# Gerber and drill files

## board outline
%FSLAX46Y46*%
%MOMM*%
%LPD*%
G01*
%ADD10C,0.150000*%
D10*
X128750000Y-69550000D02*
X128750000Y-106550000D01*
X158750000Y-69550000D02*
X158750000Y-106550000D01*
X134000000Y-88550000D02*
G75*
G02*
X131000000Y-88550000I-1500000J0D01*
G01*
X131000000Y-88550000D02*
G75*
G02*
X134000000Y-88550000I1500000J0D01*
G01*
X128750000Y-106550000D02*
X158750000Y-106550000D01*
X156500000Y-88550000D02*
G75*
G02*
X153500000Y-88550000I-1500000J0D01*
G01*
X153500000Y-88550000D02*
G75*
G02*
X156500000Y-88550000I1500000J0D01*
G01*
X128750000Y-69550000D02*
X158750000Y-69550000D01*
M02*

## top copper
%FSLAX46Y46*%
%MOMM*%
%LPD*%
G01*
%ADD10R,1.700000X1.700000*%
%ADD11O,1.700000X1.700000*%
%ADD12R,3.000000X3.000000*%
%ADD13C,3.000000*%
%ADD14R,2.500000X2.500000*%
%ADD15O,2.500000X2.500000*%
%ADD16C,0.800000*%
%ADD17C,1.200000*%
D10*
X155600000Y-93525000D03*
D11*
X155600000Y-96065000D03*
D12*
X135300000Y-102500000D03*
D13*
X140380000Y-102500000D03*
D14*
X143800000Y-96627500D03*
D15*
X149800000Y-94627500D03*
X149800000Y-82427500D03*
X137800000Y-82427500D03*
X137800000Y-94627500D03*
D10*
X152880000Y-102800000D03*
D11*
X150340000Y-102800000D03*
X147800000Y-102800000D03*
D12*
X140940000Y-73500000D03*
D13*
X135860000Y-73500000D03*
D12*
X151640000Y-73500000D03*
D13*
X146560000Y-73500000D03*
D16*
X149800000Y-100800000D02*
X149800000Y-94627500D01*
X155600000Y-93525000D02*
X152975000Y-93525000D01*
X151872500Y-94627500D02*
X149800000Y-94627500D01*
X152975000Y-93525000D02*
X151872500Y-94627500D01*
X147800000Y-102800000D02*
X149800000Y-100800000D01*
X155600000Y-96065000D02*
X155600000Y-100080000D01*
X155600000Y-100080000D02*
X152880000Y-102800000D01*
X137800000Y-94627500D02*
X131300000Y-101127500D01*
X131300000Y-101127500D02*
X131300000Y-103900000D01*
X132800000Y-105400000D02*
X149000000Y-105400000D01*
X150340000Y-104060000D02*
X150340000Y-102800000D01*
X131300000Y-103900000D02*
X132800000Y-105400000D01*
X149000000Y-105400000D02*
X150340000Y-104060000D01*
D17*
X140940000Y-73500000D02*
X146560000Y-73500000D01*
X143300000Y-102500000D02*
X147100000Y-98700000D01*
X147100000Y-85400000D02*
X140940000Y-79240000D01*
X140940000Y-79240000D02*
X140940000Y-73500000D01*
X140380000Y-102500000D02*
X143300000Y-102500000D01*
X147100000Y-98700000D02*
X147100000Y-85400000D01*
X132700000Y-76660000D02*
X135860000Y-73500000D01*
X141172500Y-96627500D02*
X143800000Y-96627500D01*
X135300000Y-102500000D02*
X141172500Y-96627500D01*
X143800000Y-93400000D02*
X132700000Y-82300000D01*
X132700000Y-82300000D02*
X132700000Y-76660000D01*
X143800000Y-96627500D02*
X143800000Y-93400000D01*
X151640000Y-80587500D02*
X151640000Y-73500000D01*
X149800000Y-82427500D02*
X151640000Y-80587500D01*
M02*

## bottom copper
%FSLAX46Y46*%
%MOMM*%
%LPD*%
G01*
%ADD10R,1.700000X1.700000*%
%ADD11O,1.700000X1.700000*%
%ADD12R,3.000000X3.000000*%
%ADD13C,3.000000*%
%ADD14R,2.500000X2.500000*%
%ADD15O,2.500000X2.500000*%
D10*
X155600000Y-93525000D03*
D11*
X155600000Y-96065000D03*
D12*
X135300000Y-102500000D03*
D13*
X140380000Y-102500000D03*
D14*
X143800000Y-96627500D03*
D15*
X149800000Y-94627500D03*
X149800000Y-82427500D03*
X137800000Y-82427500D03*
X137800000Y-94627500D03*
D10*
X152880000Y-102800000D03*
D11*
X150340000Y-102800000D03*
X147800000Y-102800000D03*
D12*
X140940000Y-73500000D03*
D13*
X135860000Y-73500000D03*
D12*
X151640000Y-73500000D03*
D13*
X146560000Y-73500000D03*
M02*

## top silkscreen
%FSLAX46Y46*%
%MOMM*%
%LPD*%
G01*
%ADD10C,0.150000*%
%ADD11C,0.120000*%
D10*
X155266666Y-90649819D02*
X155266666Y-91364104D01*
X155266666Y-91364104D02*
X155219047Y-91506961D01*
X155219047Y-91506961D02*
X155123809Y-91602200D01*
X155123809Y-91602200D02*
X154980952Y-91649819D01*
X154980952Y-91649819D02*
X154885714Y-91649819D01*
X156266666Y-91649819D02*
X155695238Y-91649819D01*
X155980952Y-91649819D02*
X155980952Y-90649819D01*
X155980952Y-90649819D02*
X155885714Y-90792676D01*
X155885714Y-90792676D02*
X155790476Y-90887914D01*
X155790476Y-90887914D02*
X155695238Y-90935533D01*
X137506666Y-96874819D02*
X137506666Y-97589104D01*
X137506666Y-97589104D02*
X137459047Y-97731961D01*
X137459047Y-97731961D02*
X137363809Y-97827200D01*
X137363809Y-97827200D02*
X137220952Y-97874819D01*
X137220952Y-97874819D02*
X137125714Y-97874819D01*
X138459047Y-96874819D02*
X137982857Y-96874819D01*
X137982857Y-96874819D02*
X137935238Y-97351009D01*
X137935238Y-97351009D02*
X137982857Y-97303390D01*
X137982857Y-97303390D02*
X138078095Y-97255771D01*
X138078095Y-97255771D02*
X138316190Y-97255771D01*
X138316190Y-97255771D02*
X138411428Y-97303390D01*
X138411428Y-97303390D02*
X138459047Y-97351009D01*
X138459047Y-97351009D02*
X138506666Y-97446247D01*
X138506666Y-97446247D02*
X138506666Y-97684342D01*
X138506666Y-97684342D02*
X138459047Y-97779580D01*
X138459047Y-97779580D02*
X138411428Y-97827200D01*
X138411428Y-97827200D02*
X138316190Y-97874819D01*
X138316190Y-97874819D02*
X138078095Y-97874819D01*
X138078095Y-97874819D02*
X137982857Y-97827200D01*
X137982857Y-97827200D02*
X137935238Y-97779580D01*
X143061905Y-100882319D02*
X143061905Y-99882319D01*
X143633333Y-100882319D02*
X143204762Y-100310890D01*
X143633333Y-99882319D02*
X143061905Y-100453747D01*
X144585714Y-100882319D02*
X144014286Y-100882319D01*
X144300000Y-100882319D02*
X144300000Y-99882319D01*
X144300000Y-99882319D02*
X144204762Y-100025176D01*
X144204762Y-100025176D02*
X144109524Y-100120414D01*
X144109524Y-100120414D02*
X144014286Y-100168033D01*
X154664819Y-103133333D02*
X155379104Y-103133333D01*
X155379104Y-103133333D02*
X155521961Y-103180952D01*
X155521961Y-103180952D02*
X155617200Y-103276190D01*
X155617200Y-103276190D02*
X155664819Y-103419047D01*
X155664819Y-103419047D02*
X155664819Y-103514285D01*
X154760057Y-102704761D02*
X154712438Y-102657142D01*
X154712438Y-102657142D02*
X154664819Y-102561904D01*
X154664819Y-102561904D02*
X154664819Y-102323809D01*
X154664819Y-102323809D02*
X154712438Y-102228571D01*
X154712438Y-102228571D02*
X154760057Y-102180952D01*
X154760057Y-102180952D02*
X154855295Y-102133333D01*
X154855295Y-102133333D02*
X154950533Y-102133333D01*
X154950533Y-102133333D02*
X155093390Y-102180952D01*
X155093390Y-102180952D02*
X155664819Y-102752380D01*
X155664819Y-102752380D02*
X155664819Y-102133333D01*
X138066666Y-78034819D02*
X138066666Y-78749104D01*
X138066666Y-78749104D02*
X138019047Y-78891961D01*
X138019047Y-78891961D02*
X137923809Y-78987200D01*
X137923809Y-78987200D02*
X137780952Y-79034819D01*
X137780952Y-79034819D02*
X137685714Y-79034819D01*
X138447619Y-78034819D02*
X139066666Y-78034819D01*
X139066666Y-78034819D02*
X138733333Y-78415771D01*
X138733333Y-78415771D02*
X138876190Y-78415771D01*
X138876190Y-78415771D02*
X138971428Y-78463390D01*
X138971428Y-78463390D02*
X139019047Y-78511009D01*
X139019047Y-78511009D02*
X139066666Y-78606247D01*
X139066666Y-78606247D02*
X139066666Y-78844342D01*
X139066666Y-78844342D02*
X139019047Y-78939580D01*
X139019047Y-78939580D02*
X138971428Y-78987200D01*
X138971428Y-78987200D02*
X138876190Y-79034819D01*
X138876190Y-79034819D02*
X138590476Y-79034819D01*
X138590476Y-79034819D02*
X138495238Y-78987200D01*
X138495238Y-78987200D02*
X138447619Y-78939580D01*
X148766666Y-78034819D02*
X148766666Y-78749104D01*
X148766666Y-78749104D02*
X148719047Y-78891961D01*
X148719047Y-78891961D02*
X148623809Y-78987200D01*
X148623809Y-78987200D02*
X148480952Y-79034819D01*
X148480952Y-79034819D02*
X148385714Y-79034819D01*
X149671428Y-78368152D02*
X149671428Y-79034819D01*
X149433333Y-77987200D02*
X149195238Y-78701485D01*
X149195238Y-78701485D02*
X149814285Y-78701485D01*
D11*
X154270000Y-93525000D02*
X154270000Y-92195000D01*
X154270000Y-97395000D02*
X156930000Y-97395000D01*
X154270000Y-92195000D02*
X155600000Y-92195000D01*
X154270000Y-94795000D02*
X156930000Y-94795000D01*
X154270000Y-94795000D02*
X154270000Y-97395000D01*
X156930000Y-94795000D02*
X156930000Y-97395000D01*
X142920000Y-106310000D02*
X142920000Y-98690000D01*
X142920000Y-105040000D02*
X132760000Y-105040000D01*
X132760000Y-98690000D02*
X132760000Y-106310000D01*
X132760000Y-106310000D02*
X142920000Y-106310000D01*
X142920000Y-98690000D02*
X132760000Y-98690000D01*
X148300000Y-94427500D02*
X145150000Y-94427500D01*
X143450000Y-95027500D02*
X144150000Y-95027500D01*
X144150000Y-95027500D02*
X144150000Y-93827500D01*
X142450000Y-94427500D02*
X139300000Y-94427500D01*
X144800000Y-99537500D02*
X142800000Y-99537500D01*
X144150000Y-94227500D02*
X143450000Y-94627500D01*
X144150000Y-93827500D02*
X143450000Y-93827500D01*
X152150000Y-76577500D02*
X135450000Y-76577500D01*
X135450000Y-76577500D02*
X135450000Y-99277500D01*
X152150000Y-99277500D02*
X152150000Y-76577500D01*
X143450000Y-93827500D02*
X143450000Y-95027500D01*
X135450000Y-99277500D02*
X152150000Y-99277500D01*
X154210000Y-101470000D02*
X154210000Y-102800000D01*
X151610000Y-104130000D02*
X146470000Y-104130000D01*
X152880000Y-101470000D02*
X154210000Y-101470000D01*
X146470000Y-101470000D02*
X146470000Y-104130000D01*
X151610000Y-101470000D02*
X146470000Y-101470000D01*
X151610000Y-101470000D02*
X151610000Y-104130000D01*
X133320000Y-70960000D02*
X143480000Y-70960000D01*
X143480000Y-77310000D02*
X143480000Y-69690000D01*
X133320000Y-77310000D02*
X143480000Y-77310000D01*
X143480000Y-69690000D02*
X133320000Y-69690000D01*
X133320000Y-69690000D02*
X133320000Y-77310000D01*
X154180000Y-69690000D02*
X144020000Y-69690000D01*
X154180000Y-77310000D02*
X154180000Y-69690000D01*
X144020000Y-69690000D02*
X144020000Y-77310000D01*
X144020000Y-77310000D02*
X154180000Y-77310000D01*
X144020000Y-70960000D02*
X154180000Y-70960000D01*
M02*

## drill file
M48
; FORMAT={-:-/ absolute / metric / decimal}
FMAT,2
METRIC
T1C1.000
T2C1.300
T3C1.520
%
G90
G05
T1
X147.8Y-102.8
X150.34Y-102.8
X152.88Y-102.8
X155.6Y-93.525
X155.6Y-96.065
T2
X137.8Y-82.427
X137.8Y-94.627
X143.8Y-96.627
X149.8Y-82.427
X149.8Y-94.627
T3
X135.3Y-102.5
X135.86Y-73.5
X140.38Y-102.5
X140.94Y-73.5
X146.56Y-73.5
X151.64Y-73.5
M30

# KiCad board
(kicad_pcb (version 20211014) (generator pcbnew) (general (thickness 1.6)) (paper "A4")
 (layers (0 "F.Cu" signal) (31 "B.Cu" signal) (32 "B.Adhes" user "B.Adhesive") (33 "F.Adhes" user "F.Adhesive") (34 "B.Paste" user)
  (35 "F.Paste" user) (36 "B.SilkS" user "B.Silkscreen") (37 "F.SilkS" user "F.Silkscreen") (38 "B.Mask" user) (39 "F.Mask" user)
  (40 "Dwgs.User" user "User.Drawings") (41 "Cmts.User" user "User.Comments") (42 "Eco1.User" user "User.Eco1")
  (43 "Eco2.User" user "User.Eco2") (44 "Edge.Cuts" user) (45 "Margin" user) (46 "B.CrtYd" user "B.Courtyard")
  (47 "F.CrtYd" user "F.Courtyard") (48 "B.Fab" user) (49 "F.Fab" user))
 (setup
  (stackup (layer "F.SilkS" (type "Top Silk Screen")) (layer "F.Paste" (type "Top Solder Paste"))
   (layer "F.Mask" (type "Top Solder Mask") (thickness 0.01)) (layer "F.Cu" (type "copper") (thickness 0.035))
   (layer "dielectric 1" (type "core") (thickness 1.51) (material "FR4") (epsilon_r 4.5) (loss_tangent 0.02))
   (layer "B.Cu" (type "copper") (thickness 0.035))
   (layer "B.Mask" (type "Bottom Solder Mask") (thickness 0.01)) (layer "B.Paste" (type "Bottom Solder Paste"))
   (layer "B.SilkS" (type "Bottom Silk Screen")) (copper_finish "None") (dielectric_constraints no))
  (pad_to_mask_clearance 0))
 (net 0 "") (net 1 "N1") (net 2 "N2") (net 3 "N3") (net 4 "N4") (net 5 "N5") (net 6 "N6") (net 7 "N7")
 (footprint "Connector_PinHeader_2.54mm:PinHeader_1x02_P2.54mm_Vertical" (layer "F.Cu") (at 155.6 93.525)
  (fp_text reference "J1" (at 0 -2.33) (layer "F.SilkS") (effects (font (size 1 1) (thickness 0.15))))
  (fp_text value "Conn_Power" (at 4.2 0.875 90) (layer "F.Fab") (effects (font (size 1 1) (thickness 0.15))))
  (fp_line (start -1.33 0) (end -1.33 -1.33) (layer "F.SilkS") (width 0.12))
  (fp_line (start -1.33 3.87) (end 1.33 3.87) (layer "F.SilkS") (width 0.12))
  (fp_line (start -1.33 -1.33) (end 0 -1.33) (layer "F.SilkS") (width 0.12))
  (fp_line (start -1.33 1.27) (end 1.33 1.27) (layer "F.SilkS") (width 0.12))
  (fp_line (start -1.33 1.27) (end -1.33 3.87) (layer "F.SilkS") (width 0.12))
  (fp_line (start 1.33 1.27) (end 1.33 3.87) (layer "F.SilkS") (width 0.12))
  (pad "1" thru_hole rect locked (at 0 0) (size 1.7 1.7) (drill 1) (layers *.Cu *.Mask) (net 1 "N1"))
  (pad "2" thru_hole oval locked (at 0 2.54) (size 1.7 1.7) (drill 1) (layers *.Cu *.Mask) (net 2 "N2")))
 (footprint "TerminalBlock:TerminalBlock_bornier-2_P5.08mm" (layer "F.Cu") (at 135.3 102.5)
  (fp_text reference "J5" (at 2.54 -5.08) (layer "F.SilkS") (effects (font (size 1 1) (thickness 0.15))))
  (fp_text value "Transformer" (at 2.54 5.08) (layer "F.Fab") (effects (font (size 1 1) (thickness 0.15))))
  (fp_line (start 7.62 3.81) (end 7.62 -3.81) (layer "F.SilkS") (width 0.12))
  (fp_line (start 7.62 2.54) (end -2.54 2.54) (layer "F.SilkS") (width 0.12))
  (fp_line (start -2.54 -3.81) (end -2.54 3.81) (layer "F.SilkS") (width 0.12))
  (fp_line (start -2.54 3.81) (end 7.62 3.81) (layer "F.SilkS") (width 0.12))
  (fp_line (start 7.62 -3.81) (end -2.54 -3.81) (layer "F.SilkS") (width 0.12))
  (pad "1" thru_hole rect locked (at 0 0) (size 3 3) (drill 1.52) (layers *.Cu *.Mask) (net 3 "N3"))
  (pad "2" thru_hole circle locked (at 5.08 0) (size 3 3) (drill 1.52) (layers *.Cu *.Mask) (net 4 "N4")))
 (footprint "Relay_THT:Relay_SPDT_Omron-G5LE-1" (layer "F.Cu") (at 143.8 96.6275 180)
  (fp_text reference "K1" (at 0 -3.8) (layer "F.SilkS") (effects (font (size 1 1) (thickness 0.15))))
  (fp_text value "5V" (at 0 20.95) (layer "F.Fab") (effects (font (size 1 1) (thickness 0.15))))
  (fp_line (start -4.5 2.2) (end -1.35 2.2) (layer "F.SilkS") (width 0.12))
  (fp_line (start 0.35 1.6) (end -0.35 1.6) (layer "F.SilkS") (width 0.12))
  (fp_line (start -0.35 1.6) (end -0.35 2.8) (layer "F.SilkS") (width 0.12))
  (fp_line (start 1.35 2.2) (end 4.5 2.2) (layer "F.SilkS") (width 0.12))
  (fp_line (start -1 -2.91) (end 1 -2.91) (layer "F.SilkS") (width 0.12))
  (fp_line (start -0.35 2.4) (end 0.35 2) (layer "F.SilkS") (width 0.12))
  (fp_line (start -0.35 2.8) (end 0.35 2.8) (layer "F.SilkS") (width 0.12))
  (fp_line (start -8.35 20.05) (end 8.35 20.05) (layer "F.SilkS") (width 0.12))
  (fp_line (start 8.35 20.05) (end 8.35 -2.65) (layer "F.SilkS") (width 0.12))
  (fp_line (start -8.35 -2.65) (end -8.35 20.05) (layer "F.SilkS") (width 0.12))
  (fp_line (start 0.35 2.8) (end 0.35 1.6) (layer "F.SilkS") (width 0.12))
  (fp_line (start 8.35 -2.65) (end -8.35 -2.65) (layer "F.SilkS") (width 0.12))
  (pad "1" thru_hole rect locked (at 0 0 180) (size 2.5 2.5) (drill 1.3) (layers *.Cu *.Mask) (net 3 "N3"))
  (pad "2" thru_hole oval locked (at -6 2 180) (size 2.5 2.5) (drill 1.3) (layers *.Cu *.Mask) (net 1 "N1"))
  (pad "3" thru_hole oval locked (at -6 14.2 180) (size 2.5 2.5) (drill 1.3) (layers *.Cu *.Mask) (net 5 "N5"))
  (pad "4" thru_hole oval locked (at 6 14.2 180) (size 2.5 2.5) (drill 1.3) (layers *.Cu *.Mask) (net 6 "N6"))
  (pad "5" thru_hole oval locked (at 6 2 180) (size 2.5 2.5) (drill 1.3) (layers *.Cu *.Mask) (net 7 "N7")))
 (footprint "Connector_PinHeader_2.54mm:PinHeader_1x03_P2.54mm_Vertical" (layer "F.Cu") (at 152.88 102.8 -90)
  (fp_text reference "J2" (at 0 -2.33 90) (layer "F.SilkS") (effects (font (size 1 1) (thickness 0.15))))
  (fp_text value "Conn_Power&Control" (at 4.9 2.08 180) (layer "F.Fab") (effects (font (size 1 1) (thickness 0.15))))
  (fp_line (start -1.33 -1.33) (end 0 -1.33) (layer "F.SilkS") (width 0.12))
  (fp_line (start 1.33 1.27) (end 1.33 6.41) (layer "F.SilkS") (width 0.12))
  (fp_line (start -1.33 0) (end -1.33 -1.33) (layer "F.SilkS") (width 0.12))
  (fp_line (start -1.33 6.41) (end 1.33 6.41) (layer "F.SilkS") (width 0.12))
  (fp_line (start -1.33 1.27) (end -1.33 6.41) (layer "F.SilkS") (width 0.12))
  (fp_line (start -1.33 1.27) (end 1.33 1.27) (layer "F.SilkS") (width 0.12))
  (pad "1" thru_hole rect locked (at 0 0 270) (size 1.7 1.7) (drill 1) (layers *.Cu *.Mask) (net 2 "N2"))
  (pad "2" thru_hole oval locked (at 0 2.54 270) (size 1.7 1.7) (drill 1) (layers *.Cu *.Mask) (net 7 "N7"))
  (pad "3" thru_hole oval locked (at 0 5.08 270) (size 1.7 1.7) (drill 1) (layers *.Cu *.Mask) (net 1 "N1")))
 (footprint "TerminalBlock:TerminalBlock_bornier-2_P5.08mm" (layer "F.Cu") (at 140.94 73.5 180)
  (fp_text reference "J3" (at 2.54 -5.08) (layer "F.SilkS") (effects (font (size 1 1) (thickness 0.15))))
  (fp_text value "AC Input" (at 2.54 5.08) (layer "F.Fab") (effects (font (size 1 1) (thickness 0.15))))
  (fp_line (start 7.62 2.54) (end -2.54 2.54) (layer "F.SilkS") (width 0.12))
  (fp_line (start -2.54 -3.81) (end -2.54 3.81) (layer "F.SilkS") (width 0.12))
  (fp_line (start 7.62 -3.81) (end -2.54 -3.81) (layer "F.SilkS") (width 0.12))
  (fp_line (start -2.54 3.81) (end 7.62 3.81) (layer "F.SilkS") (width 0.12))
  (fp_line (start 7.62 3.81) (end 7.62 -3.81) (layer "F.SilkS") (width 0.12))
  (pad "1" thru_hole rect locked (at 0 0 180) (size 3 3) (drill 1.52) (layers *.Cu *.Mask) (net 4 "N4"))
  (pad "2" thru_hole circle locked (at 5.08 0 180) (size 3 3) (drill 1.52) (layers *.Cu *.Mask) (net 3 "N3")))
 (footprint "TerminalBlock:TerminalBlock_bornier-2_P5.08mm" (layer "F.Cu") (at 151.64 73.5 180)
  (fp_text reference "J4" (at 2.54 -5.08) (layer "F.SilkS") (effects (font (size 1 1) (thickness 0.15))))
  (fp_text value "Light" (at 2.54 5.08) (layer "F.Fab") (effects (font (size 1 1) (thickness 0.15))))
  (fp_line (start -2.54 3.81) (end 7.62 3.81) (layer "F.SilkS") (width 0.12))
  (fp_line (start -2.54 -3.81) (end -2.54 3.81) (layer "F.SilkS") (width 0.12))
  (fp_line (start 7.62 3.81) (end 7.62 -3.81) (layer "F.SilkS") (width 0.12))
  (fp_line (start 7.62 -3.81) (end -2.54 -3.81) (layer "F.SilkS") (width 0.12))
  (fp_line (start 7.62 2.54) (end -2.54 2.54) (layer "F.SilkS") (width 0.12))
  (pad "1" thru_hole rect locked (at 0 0 180) (size 3 3) (drill 1.52) (layers *.Cu *.Mask) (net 5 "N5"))
  (pad "2" thru_hole circle locked (at 5.08 0 180) (size 3 3) (drill 1.52) (layers *.Cu *.Mask) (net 4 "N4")))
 (gr_line (start 128.75 69.55) (end 128.75 106.55) (layer "Edge.Cuts") (width 0.15))
 (gr_line (start 158.75 69.55) (end 158.75 106.55) (layer "Edge.Cuts") (width 0.15))
 (gr_circle (center 132.5 88.55) (end 134 88.55) (layer "Edge.Cuts") (width 0.15) (fill none))
 (gr_line (start 128.75 106.55) (end 158.75 106.55) (layer "Edge.Cuts") (width 0.15))
 (gr_circle (center 155 88.55) (end 156.5 88.55) (layer "Edge.Cuts") (width 0.15) (fill none))
 (gr_line (start 128.75 69.55) (end 158.75 69.55) (layer "Edge.Cuts") (width 0.15))
 (segment (start 149.8 100.8) (end 149.8 94.6275) (width 0.8) (layer "F.Cu") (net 1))
 (segment (start 155.6 93.525) (end 152.975 93.525) (width 0.8) (layer "F.Cu") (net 1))
 (segment (start 151.8725 94.6275) (end 149.8 94.6275) (width 0.8) (layer "F.Cu") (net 1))
 (segment (start 152.975 93.525) (end 151.8725 94.6275) (width 0.8) (layer "F.Cu") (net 1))
 (segment (start 147.8 102.8) (end 149.8 100.8) (width 0.8) (layer "F.Cu") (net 1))
 (segment (start 155.6 96.065) (end 155.6 100.08) (width 0.8) (layer "F.Cu") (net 2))
 (segment (start 155.6 100.08) (end 152.88 102.8) (width 0.8) (layer "F.Cu") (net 2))
 (segment (start 137.8 94.6275) (end 131.3 101.1275) (width 0.8) (layer "F.Cu") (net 7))
 (segment (start 131.3 101.1275) (end 131.3 103.9) (width 0.8) (layer "F.Cu") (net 7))
 (segment (start 132.8 105.4) (end 149 105.4) (width 0.8) (layer "F.Cu") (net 7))
 (segment (start 150.34 104.06) (end 150.34 102.8) (width 0.8) (layer "F.Cu") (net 7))
 (segment (start 131.3 103.9) (end 132.8 105.4) (width 0.8) (layer "F.Cu") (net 7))
 (segment (start 149 105.4) (end 150.34 104.06) (width 0.8) (layer "F.Cu") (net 7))
 (segment (start 140.94 73.5) (end 146.56 73.5) (width 1.2) (layer "F.Cu") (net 4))
 (segment (start 143.3 102.5) (end 147.1 98.7) (width 1.2) (layer "F.Cu") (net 4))
 (segment (start 147.1 85.4) (end 140.94 79.24) (width 1.2) (layer "F.Cu") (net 4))
 (segment (start 140.94 79.24) (end 140.94 73.5) (width 1.2) (layer "F.Cu") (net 4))
 (segment (start 140.38 102.5) (end 143.3 102.5) (width 1.2) (layer "F.Cu") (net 4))
 (segment (start 147.1 98.7) (end 147.1 85.4) (width 1.2) (layer "F.Cu") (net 4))
 (segment (start 132.7 76.66) (end 135.86 73.5) (width 1.2) (layer "F.Cu") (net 3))
 (segment (start 141.1725 96.6275) (end 143.8 96.6275) (width 1.2) (layer "F.Cu") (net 3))
 (segment (start 135.3 102.5) (end 141.1725 96.6275) (width 1.2) (layer "F.Cu") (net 3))
 (segment (start 143.8 93.4) (end 132.7 82.3) (width 1.2) (layer "F.Cu") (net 3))
 (segment (start 132.7 82.3) (end 132.7 76.66) (width 1.2) (layer "F.Cu") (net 3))
 (segment (start 143.8 96.6275) (end 143.8 93.4) (width 1.2) (layer "F.Cu") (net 3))
 (segment (start 151.64 80.5875) (end 151.64 73.5) (width 1.2) (layer "F.Cu") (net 5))
 (segment (start 149.8 82.4275) (end 151.64 80.5875) (width 1.2) (layer "F.Cu") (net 5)))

